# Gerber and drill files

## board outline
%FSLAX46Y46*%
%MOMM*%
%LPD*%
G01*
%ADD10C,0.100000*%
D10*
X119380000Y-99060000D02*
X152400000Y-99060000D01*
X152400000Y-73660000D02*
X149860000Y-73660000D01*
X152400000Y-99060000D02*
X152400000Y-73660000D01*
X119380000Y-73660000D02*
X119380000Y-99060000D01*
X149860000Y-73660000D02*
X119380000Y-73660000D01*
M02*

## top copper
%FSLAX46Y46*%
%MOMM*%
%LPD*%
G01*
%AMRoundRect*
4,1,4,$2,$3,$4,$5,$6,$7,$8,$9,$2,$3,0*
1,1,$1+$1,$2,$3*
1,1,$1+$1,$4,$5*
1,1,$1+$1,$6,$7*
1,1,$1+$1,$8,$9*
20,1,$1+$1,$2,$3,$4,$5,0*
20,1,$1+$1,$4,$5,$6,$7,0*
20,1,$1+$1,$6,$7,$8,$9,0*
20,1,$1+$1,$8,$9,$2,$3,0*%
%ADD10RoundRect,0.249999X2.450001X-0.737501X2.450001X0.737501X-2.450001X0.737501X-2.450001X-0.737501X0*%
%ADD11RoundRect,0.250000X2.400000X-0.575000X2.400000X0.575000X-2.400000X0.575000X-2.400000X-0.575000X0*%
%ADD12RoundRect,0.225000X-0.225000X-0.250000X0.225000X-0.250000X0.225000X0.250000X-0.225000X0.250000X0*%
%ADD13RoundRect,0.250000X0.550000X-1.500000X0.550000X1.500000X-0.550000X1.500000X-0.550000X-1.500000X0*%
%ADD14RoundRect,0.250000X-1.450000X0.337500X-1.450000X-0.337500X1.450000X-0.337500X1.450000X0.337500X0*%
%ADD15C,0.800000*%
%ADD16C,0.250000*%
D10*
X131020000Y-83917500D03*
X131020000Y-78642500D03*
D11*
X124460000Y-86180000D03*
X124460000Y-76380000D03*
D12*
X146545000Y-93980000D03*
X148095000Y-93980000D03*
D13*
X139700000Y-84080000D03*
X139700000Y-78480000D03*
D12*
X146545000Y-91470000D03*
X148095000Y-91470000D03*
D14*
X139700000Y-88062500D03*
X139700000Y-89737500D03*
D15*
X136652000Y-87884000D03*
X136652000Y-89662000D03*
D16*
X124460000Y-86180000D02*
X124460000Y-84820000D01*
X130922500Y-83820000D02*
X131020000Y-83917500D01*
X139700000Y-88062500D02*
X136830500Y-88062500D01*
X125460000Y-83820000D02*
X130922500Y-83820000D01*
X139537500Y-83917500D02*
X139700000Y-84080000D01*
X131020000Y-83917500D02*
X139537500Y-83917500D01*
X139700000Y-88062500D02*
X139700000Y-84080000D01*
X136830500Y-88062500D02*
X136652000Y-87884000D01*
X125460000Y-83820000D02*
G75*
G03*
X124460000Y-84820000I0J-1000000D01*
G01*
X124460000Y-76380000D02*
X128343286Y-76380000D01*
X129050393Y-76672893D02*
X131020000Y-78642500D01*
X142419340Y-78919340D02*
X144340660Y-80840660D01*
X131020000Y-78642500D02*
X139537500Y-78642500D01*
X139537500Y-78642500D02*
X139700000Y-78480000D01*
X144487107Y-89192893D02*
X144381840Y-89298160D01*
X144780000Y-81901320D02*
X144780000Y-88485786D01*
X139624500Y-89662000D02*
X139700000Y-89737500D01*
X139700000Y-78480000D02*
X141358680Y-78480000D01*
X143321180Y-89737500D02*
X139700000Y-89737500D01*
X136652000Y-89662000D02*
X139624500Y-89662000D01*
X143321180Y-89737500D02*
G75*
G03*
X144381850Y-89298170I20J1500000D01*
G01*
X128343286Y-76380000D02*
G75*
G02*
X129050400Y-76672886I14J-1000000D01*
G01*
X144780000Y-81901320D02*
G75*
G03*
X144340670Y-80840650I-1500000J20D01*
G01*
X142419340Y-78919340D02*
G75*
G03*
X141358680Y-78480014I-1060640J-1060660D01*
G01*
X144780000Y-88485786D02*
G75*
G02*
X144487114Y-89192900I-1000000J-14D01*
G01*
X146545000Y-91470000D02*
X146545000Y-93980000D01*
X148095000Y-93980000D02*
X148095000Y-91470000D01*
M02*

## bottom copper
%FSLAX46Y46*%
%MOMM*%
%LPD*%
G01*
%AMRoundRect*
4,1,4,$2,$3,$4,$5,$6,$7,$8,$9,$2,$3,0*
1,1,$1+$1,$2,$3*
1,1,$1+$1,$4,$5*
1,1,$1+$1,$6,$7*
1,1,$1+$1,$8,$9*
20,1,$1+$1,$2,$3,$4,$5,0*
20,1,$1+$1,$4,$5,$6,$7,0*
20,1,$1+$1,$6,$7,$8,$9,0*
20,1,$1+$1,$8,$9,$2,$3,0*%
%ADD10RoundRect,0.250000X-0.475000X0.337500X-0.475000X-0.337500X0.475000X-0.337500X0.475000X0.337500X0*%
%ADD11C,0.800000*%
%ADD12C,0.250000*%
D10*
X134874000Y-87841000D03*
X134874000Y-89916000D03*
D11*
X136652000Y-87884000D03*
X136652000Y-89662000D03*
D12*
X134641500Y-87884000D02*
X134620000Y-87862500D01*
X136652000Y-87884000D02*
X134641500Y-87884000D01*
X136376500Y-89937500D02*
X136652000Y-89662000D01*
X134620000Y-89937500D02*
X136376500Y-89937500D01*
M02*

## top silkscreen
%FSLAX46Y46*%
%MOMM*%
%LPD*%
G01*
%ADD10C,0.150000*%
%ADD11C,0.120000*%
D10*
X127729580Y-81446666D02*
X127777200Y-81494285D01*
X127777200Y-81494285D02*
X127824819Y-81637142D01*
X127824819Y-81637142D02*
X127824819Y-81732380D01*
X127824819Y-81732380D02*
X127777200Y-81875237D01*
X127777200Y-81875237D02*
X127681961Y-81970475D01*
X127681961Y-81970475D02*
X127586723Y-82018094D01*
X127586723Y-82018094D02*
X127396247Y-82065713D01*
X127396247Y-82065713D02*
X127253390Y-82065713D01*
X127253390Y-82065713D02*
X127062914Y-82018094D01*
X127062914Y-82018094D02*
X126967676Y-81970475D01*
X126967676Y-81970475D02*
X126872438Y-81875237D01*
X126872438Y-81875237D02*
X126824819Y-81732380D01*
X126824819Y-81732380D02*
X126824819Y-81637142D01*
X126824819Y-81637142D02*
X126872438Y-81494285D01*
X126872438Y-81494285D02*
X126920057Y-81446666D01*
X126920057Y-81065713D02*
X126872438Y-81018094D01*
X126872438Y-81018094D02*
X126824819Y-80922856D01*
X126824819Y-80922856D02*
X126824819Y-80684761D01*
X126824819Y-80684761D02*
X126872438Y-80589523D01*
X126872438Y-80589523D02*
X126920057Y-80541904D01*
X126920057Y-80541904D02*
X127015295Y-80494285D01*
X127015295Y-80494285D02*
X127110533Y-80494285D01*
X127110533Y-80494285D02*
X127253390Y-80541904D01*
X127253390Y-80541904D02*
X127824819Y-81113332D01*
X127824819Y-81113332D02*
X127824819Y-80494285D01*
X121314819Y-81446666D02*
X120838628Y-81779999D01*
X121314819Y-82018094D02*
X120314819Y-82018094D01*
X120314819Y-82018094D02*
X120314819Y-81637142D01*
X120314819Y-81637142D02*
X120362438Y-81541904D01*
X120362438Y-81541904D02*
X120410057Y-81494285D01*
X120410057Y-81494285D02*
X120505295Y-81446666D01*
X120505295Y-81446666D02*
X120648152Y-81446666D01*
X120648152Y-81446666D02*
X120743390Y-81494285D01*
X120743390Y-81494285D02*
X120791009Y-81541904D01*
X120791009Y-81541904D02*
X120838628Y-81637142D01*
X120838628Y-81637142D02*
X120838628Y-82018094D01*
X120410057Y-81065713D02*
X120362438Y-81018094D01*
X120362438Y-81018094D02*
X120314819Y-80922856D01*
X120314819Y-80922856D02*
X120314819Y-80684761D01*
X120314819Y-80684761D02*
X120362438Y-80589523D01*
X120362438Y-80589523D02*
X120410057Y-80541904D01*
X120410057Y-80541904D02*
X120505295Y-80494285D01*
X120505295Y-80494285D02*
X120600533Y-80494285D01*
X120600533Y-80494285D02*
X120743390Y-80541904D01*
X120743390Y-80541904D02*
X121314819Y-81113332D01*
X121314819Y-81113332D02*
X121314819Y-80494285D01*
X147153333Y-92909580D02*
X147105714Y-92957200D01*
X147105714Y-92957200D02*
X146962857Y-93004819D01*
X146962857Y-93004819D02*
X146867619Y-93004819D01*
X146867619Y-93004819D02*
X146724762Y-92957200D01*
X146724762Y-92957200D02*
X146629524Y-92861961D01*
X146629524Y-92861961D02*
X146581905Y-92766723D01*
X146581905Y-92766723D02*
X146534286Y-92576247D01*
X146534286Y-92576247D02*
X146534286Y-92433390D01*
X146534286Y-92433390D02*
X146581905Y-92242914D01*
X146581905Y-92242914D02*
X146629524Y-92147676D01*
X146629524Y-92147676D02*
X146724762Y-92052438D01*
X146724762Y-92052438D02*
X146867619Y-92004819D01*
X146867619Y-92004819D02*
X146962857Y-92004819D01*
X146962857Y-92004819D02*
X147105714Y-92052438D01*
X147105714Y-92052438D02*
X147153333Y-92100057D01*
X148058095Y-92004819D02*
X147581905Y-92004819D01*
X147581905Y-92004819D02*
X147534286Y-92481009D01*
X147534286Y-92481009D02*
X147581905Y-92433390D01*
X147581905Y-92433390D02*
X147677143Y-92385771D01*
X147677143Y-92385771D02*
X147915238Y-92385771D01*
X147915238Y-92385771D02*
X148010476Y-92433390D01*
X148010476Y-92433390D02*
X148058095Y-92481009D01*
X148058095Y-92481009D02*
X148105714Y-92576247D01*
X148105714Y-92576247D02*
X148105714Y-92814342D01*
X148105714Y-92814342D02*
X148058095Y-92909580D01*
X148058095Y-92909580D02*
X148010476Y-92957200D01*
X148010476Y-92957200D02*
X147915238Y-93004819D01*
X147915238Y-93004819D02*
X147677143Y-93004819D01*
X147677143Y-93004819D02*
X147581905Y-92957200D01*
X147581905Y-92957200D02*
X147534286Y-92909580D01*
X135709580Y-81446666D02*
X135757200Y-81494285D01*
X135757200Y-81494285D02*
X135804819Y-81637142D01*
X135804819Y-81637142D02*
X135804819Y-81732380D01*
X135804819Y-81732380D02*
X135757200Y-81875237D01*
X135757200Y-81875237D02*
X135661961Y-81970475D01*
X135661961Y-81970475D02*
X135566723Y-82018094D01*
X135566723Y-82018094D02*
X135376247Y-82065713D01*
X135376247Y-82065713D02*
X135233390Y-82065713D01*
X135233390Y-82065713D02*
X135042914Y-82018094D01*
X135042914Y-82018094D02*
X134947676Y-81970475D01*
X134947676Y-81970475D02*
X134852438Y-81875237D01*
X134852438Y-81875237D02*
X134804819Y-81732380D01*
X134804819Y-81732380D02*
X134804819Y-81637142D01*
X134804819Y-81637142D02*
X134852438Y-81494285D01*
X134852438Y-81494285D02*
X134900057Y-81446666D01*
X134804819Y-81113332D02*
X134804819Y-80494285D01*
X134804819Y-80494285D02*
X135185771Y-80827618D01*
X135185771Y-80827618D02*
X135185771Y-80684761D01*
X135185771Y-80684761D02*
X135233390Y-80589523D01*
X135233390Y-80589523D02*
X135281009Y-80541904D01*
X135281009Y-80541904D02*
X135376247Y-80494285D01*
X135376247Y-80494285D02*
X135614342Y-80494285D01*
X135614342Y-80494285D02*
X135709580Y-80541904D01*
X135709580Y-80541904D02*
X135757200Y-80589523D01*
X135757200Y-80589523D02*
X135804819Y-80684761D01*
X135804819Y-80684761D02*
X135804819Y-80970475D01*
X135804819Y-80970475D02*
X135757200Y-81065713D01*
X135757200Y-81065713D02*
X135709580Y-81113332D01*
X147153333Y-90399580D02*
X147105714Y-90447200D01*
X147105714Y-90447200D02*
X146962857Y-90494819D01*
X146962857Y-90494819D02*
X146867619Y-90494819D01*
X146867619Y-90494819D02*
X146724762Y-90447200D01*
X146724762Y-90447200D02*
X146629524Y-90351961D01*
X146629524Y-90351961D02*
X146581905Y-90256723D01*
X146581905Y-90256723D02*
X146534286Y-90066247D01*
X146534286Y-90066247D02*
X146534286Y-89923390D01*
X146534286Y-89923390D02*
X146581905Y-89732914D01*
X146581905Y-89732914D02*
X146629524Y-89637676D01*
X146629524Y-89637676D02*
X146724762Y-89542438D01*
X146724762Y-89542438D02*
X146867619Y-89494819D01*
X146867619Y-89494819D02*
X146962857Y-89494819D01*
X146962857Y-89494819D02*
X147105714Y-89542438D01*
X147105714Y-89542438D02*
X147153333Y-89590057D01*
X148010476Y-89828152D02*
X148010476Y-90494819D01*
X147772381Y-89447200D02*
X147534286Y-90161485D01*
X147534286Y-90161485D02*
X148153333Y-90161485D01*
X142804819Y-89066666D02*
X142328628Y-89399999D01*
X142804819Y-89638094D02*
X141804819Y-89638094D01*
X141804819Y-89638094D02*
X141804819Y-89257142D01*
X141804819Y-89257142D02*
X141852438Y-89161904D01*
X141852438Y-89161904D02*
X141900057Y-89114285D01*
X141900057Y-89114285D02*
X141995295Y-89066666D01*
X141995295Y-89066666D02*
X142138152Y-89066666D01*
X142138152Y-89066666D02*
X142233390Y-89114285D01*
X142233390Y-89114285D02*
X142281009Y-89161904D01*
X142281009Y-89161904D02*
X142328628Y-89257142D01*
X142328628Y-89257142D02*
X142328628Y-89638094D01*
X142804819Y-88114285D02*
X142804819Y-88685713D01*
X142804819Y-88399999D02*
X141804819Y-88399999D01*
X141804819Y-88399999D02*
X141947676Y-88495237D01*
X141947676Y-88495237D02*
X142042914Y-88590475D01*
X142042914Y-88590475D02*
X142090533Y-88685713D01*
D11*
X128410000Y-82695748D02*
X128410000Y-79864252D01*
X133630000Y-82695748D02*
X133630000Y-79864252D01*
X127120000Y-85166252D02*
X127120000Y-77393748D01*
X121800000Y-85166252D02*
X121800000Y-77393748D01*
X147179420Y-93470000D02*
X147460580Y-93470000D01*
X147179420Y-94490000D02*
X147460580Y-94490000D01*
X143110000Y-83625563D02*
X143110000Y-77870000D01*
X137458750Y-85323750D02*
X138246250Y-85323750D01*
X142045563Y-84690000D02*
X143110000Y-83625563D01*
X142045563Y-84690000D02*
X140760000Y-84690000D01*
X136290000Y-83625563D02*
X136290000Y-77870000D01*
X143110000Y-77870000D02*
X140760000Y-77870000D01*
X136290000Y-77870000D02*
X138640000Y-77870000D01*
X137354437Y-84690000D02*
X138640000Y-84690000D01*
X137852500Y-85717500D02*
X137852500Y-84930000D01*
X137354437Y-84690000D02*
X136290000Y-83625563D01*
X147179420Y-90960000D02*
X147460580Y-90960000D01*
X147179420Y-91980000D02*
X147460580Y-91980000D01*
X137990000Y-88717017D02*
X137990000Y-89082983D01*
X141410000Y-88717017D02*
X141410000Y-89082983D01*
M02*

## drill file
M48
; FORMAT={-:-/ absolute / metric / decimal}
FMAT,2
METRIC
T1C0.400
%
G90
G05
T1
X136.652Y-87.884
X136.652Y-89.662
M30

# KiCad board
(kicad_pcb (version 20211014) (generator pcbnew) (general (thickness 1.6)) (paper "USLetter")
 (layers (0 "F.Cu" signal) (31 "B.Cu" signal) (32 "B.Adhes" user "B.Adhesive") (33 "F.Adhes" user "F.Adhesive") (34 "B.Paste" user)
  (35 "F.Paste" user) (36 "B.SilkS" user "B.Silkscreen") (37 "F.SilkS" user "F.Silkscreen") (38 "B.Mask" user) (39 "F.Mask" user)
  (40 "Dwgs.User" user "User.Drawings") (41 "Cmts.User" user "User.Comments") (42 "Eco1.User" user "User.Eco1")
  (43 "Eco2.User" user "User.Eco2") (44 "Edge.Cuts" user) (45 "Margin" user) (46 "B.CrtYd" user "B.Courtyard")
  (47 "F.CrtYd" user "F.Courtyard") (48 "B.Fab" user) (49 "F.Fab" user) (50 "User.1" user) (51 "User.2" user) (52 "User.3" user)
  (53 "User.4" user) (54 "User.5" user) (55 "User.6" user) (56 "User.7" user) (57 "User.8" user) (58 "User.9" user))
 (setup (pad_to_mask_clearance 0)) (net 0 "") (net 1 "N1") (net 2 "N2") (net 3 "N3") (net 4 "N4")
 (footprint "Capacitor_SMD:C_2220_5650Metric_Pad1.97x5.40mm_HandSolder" (layer "F.Cu") (at 131.02 81.28 90)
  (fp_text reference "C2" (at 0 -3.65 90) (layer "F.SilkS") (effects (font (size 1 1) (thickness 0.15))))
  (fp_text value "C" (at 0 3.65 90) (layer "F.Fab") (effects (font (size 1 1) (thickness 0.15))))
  (fp_line (start -1.415748 -2.61) (end 1.415748 -2.61) (layer "F.SilkS") (width 0.12))
  (fp_line (start -1.415748 2.61) (end 1.415748 2.61) (layer "F.SilkS") (width 0.12))
  (pad "1" smd roundrect (at -2.6375 0 90) (size 1.975 5.4) (layers "F.Cu" "F.Paste" "F.Mask") (roundrect_rratio 0.126582) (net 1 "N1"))
  (pad "2" smd roundrect (at 2.6375 0 90) (size 1.975 5.4) (layers "F.Cu" "F.Paste" "F.Mask") (roundrect_rratio 0.126582) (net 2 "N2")))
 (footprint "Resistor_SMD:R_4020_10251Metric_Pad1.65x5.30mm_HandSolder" (layer "F.Cu") (at 124.46 81.28 90)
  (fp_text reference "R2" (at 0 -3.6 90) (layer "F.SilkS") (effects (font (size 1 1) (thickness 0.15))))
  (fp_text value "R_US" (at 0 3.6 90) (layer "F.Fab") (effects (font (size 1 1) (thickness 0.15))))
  (fp_line (start -3.886252 2.66) (end 3.886252 2.66) (layer "F.SilkS") (width 0.12))
  (fp_line (start -3.886252 -2.66) (end 3.886252 -2.66) (layer "F.SilkS") (width 0.12))
  (pad "1" smd roundrect (at -4.9 0 90) (size 1.65 5.3) (layers "F.Cu" "F.Paste" "F.Mask") (roundrect_rratio 0.151515) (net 1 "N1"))
  (pad "2" smd roundrect (at 4.9 0 90) (size 1.65 5.3) (layers "F.Cu" "F.Paste" "F.Mask") (roundrect_rratio 0.151515) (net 2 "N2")))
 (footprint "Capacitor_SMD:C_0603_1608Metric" (layer "F.Cu") (at 147.32 93.98)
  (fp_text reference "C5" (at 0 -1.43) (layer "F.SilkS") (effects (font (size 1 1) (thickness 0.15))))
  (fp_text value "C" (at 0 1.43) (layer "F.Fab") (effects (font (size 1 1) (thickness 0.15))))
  (fp_line (start -0.14058 -0.51) (end 0.14058 -0.51) (layer "F.SilkS") (width 0.12))
  (fp_line (start -0.14058 0.51) (end 0.14058 0.51) (layer "F.SilkS") (width 0.12))
  (pad "1" smd roundrect (at -0.775 0) (size 0.9 0.95) (layers "F.Cu" "F.Paste" "F.Mask") (roundrect_rratio 0.25) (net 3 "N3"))
  (pad "2" smd roundrect (at 0.775 0) (size 0.9 0.95) (layers "F.Cu" "F.Paste" "F.Mask") (roundrect_rratio 0.25) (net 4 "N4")))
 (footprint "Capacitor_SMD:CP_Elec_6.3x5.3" (layer "F.Cu") (at 139.7 81.28 90)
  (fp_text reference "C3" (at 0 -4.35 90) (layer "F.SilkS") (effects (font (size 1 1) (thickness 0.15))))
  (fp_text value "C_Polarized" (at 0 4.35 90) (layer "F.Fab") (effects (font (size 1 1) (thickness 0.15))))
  (fp_line (start -2.345563 3.41) (end 3.41 3.41) (layer "F.SilkS") (width 0.12))
  (fp_line (start -4.04375 -2.24125) (end -4.04375 -1.45375) (layer "F.SilkS") (width 0.12))
  (fp_line (start -3.41 2.345563) (end -2.345563 3.41) (layer "F.SilkS") (width 0.12))
  (fp_line (start -3.41 2.345563) (end -3.41 1.06) (layer "F.SilkS") (width 0.12))
  (fp_line (start -2.345563 -3.41) (end 3.41 -3.41) (layer "F.SilkS") (width 0.12))
  (fp_line (start 3.41 3.41) (end 3.41 1.06) (layer "F.SilkS") (width 0.12))
  (fp_line (start 3.41 -3.41) (end 3.41 -1.06) (layer "F.SilkS") (width 0.12))
  (fp_line (start -3.41 -2.345563) (end -3.41 -1.06) (layer "F.SilkS") (width 0.12))
  (fp_line (start -4.4375 -1.8475) (end -3.65 -1.8475) (layer "F.SilkS") (width 0.12))
  (fp_line (start -3.41 -2.345563) (end -2.345563 -3.41) (layer "F.SilkS") (width 0.12))
  (pad "1" smd roundrect (at -2.8 0 90) (size 3.5 1.6) (layers "F.Cu" "F.Paste" "F.Mask") (roundrect_rratio 0.15625) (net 1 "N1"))
  (pad "2" smd roundrect (at 2.8 0 90) (size 3.5 1.6) (layers "F.Cu" "F.Paste" "F.Mask") (roundrect_rratio 0.15625) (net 2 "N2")))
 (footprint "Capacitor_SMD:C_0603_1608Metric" (layer "F.Cu") (at 147.32 91.47)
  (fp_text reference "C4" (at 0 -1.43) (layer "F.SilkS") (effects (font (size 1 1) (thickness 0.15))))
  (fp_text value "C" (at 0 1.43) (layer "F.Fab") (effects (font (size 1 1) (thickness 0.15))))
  (fp_line (start -0.14058 -0.51) (end 0.14058 -0.51) (layer "F.SilkS") (width 0.12))
  (fp_line (start -0.14058 0.51) (end 0.14058 0.51) (layer "F.SilkS") (width 0.12))
  (pad "1" smd roundrect (at -0.775 0) (size 0.9 0.95) (layers "F.Cu" "F.Paste" "F.Mask") (roundrect_rratio 0.25) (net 3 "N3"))
  (pad "2" smd roundrect (at 0.775 0) (size 0.9 0.95) (layers "F.Cu" "F.Paste" "F.Mask") (roundrect_rratio 0.25) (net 4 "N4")))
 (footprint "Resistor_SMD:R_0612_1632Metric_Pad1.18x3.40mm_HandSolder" (layer "F.Cu") (at 139.7 88.9 -90)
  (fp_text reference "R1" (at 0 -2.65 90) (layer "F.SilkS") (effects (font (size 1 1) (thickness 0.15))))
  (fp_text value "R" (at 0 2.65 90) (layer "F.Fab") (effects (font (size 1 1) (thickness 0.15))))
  (fp_line (start -0.182983 1.71) (end 0.182983 1.71) (layer "F.SilkS") (width 0.12))
  (fp_line (start -0.182983 -1.71) (end 0.182983 -1.71) (layer "F.SilkS") (width 0.12))
  (pad "1" smd roundrect (at -0.8375 0 270) (size 1.175 3.4) (layers "F.Cu" "F.Paste" "F.Mask") (roundrect_rratio 0.212766) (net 1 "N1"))
  (pad "2" smd roundrect (at 0.8375 0 270) (size 1.175 3.4) (layers "F.Cu" "F.Paste" "F.Mask") (roundrect_rratio 0.212766) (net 2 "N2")))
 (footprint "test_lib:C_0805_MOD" (layer "B.Cu") (at 134.874 88.8785 -90)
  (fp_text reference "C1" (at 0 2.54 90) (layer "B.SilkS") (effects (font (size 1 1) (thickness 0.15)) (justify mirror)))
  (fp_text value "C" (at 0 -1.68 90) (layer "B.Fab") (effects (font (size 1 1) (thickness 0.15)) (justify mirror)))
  (pad "1" smd roundrect (at -1.0375 0 270) (size 1.175 1.45) (layers "B.Cu" "B.Paste" "B.Mask") (roundrect_rratio 0.212766) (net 1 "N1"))
  (pad "2" smd roundrect (at 1.0375 0 270) (size 1.175 1.45) (layers "B.Cu" "B.Paste" "B.Mask") (roundrect_rratio 0.212766) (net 2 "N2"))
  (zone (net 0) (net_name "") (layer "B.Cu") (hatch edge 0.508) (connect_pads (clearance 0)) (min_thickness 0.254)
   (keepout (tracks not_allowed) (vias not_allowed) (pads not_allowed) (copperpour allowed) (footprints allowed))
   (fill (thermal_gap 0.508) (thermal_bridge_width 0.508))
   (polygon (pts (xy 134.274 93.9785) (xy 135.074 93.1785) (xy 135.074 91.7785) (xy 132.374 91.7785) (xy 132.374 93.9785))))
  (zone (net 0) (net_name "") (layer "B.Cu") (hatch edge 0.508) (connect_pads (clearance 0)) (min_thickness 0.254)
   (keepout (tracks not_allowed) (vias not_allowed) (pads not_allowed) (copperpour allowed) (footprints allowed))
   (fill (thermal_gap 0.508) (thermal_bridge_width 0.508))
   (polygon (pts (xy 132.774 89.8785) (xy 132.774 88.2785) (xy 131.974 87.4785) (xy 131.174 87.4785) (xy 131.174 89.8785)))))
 (gr_line (start 119.38 99.06) (end 152.4 99.06) (layer "Edge.Cuts") (width 0.1))
 (gr_line (start 152.4 73.66) (end 149.86 73.66) (layer "Edge.Cuts") (width 0.1))
 (gr_line (start 152.4 99.06) (end 152.4 73.66) (layer "Edge.Cuts") (width 0.1))
 (gr_line (start 119.38 73.66) (end 119.38 99.06) (layer "Edge.Cuts") (width 0.1))
 (gr_line (start 149.86 73.66) (end 119.38 73.66) (layer "Edge.Cuts") (width 0.1))
 (segment (start 124.46 86.18) (end 124.46 84.82) (width 0.25) (layer "F.Cu") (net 1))
 (segment (start 130.9225 83.82) (end 131.02 83.9175) (width 0.25) (layer "F.Cu") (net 1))
 (segment (start 139.7 88.0625) (end 136.8305 88.0625) (width 0.25) (layer "F.Cu") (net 1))
 (segment (start 125.46 83.82) (end 130.9225 83.82) (width 0.25) (layer "F.Cu") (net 1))
 (segment (start 139.5375 83.9175) (end 139.7 84.08) (width 0.25) (layer "F.Cu") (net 1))
 (segment (start 131.02 83.9175) (end 139.5375 83.9175) (width 0.25) (layer "F.Cu") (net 1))
 (segment (start 139.7 88.0625) (end 139.7 84.08) (width 0.25) (layer "F.Cu") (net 1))
 (segment (start 136.8305 88.0625) (end 136.652 87.884) (width 0.25) (layer "F.Cu") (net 1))
 (via (at 136.652 87.884) (size 0.8) (drill 0.4) (layers "F.Cu" "B.Cu") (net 1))
 (arc (start 125.46 83.82) (mid 124.752893 84.112893) (end 124.46 84.82) (width 0.25) (layer "F.Cu") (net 1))
 (segment (start 134.6415 87.884) (end 134.62 87.8625) (width 0.25) (layer "B.Cu") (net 1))
 (segment (start 136.652 87.884) (end 134.6415 87.884) (width 0.25) (layer "B.Cu") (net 1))
 (segment (start 124.46 76.38) (end 128.343286 76.38) (width 0.25) (layer "F.Cu") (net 2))
 (segment (start 129.050393 76.672893) (end 131.02 78.6425) (width 0.25) (layer "F.Cu") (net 2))
 (segment (start 142.41934 78.91934) (end 144.34066 80.84066) (width 0.25) (layer "F.Cu") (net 2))
 (segment (start 131.02 78.6425) (end 139.5375 78.6425) (width 0.25) (layer "F.Cu") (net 2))
 (segment (start 139.5375 78.6425) (end 139.7 78.48) (width 0.25) (layer "F.Cu") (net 2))
 (segment (start 144.487107 89.192893) (end 144.38184 89.29816) (width 0.25) (layer "F.Cu") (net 2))
 (segment (start 144.78 81.90132) (end 144.78 88.485786) (width 0.25) (layer "F.Cu") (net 2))
 (segment (start 139.6245 89.662) (end 139.7 89.7375) (width 0.25) (layer "F.Cu") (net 2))
 (segment (start 139.7 78.48) (end 141.35868 78.48) (width 0.25) (layer "F.Cu") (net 2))
 (segment (start 143.32118 89.7375) (end 139.7 89.7375) (width 0.25) (layer "F.Cu") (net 2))
 (segment (start 136.652 89.662) (end 139.6245 89.662) (width 0.25) (layer "F.Cu") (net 2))
 (via (at 136.652 89.662) (size 0.8) (drill 0.4) (layers "F.Cu" "B.Cu") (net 2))
 (arc (start 143.32118 89.7375) (mid 143.895205 89.623319) (end 144.38184 89.29816) (width 0.25) (layer "F.Cu") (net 2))
 (arc (start 128.343286 76.38) (mid 128.725969 76.45612) (end 129.050393 76.672893) (width 0.25) (layer "F.Cu") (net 2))
 (arc (start 144.78 81.90132) (mid 144.665819 81.327295) (end 144.34066 80.84066) (width 0.25) (layer "F.Cu") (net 2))
 (arc (start 142.41934 78.91934) (mid 141.932705 78.594181) (end 141.35868 78.48) (width 0.25) (layer "F.Cu") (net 2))
 (arc (start 144.78 88.485786) (mid 144.70388 88.868469) (end 144.487107 89.192893) (width 0.25) (layer "F.Cu") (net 2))
 (segment (start 136.3765 89.9375) (end 136.652 89.662) (width 0.25) (layer "B.Cu") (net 2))
 (segment (start 134.62 89.9375) (end 136.3765 89.9375) (width 0.25) (layer "B.Cu") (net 2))
 (segment (start 146.545 91.47) (end 146.545 93.98) (width 0.25) (layer "F.Cu") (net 3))
 (segment (start 148.095 93.98) (end 148.095 91.47) (width 0.25) (layer "F.Cu") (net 4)))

